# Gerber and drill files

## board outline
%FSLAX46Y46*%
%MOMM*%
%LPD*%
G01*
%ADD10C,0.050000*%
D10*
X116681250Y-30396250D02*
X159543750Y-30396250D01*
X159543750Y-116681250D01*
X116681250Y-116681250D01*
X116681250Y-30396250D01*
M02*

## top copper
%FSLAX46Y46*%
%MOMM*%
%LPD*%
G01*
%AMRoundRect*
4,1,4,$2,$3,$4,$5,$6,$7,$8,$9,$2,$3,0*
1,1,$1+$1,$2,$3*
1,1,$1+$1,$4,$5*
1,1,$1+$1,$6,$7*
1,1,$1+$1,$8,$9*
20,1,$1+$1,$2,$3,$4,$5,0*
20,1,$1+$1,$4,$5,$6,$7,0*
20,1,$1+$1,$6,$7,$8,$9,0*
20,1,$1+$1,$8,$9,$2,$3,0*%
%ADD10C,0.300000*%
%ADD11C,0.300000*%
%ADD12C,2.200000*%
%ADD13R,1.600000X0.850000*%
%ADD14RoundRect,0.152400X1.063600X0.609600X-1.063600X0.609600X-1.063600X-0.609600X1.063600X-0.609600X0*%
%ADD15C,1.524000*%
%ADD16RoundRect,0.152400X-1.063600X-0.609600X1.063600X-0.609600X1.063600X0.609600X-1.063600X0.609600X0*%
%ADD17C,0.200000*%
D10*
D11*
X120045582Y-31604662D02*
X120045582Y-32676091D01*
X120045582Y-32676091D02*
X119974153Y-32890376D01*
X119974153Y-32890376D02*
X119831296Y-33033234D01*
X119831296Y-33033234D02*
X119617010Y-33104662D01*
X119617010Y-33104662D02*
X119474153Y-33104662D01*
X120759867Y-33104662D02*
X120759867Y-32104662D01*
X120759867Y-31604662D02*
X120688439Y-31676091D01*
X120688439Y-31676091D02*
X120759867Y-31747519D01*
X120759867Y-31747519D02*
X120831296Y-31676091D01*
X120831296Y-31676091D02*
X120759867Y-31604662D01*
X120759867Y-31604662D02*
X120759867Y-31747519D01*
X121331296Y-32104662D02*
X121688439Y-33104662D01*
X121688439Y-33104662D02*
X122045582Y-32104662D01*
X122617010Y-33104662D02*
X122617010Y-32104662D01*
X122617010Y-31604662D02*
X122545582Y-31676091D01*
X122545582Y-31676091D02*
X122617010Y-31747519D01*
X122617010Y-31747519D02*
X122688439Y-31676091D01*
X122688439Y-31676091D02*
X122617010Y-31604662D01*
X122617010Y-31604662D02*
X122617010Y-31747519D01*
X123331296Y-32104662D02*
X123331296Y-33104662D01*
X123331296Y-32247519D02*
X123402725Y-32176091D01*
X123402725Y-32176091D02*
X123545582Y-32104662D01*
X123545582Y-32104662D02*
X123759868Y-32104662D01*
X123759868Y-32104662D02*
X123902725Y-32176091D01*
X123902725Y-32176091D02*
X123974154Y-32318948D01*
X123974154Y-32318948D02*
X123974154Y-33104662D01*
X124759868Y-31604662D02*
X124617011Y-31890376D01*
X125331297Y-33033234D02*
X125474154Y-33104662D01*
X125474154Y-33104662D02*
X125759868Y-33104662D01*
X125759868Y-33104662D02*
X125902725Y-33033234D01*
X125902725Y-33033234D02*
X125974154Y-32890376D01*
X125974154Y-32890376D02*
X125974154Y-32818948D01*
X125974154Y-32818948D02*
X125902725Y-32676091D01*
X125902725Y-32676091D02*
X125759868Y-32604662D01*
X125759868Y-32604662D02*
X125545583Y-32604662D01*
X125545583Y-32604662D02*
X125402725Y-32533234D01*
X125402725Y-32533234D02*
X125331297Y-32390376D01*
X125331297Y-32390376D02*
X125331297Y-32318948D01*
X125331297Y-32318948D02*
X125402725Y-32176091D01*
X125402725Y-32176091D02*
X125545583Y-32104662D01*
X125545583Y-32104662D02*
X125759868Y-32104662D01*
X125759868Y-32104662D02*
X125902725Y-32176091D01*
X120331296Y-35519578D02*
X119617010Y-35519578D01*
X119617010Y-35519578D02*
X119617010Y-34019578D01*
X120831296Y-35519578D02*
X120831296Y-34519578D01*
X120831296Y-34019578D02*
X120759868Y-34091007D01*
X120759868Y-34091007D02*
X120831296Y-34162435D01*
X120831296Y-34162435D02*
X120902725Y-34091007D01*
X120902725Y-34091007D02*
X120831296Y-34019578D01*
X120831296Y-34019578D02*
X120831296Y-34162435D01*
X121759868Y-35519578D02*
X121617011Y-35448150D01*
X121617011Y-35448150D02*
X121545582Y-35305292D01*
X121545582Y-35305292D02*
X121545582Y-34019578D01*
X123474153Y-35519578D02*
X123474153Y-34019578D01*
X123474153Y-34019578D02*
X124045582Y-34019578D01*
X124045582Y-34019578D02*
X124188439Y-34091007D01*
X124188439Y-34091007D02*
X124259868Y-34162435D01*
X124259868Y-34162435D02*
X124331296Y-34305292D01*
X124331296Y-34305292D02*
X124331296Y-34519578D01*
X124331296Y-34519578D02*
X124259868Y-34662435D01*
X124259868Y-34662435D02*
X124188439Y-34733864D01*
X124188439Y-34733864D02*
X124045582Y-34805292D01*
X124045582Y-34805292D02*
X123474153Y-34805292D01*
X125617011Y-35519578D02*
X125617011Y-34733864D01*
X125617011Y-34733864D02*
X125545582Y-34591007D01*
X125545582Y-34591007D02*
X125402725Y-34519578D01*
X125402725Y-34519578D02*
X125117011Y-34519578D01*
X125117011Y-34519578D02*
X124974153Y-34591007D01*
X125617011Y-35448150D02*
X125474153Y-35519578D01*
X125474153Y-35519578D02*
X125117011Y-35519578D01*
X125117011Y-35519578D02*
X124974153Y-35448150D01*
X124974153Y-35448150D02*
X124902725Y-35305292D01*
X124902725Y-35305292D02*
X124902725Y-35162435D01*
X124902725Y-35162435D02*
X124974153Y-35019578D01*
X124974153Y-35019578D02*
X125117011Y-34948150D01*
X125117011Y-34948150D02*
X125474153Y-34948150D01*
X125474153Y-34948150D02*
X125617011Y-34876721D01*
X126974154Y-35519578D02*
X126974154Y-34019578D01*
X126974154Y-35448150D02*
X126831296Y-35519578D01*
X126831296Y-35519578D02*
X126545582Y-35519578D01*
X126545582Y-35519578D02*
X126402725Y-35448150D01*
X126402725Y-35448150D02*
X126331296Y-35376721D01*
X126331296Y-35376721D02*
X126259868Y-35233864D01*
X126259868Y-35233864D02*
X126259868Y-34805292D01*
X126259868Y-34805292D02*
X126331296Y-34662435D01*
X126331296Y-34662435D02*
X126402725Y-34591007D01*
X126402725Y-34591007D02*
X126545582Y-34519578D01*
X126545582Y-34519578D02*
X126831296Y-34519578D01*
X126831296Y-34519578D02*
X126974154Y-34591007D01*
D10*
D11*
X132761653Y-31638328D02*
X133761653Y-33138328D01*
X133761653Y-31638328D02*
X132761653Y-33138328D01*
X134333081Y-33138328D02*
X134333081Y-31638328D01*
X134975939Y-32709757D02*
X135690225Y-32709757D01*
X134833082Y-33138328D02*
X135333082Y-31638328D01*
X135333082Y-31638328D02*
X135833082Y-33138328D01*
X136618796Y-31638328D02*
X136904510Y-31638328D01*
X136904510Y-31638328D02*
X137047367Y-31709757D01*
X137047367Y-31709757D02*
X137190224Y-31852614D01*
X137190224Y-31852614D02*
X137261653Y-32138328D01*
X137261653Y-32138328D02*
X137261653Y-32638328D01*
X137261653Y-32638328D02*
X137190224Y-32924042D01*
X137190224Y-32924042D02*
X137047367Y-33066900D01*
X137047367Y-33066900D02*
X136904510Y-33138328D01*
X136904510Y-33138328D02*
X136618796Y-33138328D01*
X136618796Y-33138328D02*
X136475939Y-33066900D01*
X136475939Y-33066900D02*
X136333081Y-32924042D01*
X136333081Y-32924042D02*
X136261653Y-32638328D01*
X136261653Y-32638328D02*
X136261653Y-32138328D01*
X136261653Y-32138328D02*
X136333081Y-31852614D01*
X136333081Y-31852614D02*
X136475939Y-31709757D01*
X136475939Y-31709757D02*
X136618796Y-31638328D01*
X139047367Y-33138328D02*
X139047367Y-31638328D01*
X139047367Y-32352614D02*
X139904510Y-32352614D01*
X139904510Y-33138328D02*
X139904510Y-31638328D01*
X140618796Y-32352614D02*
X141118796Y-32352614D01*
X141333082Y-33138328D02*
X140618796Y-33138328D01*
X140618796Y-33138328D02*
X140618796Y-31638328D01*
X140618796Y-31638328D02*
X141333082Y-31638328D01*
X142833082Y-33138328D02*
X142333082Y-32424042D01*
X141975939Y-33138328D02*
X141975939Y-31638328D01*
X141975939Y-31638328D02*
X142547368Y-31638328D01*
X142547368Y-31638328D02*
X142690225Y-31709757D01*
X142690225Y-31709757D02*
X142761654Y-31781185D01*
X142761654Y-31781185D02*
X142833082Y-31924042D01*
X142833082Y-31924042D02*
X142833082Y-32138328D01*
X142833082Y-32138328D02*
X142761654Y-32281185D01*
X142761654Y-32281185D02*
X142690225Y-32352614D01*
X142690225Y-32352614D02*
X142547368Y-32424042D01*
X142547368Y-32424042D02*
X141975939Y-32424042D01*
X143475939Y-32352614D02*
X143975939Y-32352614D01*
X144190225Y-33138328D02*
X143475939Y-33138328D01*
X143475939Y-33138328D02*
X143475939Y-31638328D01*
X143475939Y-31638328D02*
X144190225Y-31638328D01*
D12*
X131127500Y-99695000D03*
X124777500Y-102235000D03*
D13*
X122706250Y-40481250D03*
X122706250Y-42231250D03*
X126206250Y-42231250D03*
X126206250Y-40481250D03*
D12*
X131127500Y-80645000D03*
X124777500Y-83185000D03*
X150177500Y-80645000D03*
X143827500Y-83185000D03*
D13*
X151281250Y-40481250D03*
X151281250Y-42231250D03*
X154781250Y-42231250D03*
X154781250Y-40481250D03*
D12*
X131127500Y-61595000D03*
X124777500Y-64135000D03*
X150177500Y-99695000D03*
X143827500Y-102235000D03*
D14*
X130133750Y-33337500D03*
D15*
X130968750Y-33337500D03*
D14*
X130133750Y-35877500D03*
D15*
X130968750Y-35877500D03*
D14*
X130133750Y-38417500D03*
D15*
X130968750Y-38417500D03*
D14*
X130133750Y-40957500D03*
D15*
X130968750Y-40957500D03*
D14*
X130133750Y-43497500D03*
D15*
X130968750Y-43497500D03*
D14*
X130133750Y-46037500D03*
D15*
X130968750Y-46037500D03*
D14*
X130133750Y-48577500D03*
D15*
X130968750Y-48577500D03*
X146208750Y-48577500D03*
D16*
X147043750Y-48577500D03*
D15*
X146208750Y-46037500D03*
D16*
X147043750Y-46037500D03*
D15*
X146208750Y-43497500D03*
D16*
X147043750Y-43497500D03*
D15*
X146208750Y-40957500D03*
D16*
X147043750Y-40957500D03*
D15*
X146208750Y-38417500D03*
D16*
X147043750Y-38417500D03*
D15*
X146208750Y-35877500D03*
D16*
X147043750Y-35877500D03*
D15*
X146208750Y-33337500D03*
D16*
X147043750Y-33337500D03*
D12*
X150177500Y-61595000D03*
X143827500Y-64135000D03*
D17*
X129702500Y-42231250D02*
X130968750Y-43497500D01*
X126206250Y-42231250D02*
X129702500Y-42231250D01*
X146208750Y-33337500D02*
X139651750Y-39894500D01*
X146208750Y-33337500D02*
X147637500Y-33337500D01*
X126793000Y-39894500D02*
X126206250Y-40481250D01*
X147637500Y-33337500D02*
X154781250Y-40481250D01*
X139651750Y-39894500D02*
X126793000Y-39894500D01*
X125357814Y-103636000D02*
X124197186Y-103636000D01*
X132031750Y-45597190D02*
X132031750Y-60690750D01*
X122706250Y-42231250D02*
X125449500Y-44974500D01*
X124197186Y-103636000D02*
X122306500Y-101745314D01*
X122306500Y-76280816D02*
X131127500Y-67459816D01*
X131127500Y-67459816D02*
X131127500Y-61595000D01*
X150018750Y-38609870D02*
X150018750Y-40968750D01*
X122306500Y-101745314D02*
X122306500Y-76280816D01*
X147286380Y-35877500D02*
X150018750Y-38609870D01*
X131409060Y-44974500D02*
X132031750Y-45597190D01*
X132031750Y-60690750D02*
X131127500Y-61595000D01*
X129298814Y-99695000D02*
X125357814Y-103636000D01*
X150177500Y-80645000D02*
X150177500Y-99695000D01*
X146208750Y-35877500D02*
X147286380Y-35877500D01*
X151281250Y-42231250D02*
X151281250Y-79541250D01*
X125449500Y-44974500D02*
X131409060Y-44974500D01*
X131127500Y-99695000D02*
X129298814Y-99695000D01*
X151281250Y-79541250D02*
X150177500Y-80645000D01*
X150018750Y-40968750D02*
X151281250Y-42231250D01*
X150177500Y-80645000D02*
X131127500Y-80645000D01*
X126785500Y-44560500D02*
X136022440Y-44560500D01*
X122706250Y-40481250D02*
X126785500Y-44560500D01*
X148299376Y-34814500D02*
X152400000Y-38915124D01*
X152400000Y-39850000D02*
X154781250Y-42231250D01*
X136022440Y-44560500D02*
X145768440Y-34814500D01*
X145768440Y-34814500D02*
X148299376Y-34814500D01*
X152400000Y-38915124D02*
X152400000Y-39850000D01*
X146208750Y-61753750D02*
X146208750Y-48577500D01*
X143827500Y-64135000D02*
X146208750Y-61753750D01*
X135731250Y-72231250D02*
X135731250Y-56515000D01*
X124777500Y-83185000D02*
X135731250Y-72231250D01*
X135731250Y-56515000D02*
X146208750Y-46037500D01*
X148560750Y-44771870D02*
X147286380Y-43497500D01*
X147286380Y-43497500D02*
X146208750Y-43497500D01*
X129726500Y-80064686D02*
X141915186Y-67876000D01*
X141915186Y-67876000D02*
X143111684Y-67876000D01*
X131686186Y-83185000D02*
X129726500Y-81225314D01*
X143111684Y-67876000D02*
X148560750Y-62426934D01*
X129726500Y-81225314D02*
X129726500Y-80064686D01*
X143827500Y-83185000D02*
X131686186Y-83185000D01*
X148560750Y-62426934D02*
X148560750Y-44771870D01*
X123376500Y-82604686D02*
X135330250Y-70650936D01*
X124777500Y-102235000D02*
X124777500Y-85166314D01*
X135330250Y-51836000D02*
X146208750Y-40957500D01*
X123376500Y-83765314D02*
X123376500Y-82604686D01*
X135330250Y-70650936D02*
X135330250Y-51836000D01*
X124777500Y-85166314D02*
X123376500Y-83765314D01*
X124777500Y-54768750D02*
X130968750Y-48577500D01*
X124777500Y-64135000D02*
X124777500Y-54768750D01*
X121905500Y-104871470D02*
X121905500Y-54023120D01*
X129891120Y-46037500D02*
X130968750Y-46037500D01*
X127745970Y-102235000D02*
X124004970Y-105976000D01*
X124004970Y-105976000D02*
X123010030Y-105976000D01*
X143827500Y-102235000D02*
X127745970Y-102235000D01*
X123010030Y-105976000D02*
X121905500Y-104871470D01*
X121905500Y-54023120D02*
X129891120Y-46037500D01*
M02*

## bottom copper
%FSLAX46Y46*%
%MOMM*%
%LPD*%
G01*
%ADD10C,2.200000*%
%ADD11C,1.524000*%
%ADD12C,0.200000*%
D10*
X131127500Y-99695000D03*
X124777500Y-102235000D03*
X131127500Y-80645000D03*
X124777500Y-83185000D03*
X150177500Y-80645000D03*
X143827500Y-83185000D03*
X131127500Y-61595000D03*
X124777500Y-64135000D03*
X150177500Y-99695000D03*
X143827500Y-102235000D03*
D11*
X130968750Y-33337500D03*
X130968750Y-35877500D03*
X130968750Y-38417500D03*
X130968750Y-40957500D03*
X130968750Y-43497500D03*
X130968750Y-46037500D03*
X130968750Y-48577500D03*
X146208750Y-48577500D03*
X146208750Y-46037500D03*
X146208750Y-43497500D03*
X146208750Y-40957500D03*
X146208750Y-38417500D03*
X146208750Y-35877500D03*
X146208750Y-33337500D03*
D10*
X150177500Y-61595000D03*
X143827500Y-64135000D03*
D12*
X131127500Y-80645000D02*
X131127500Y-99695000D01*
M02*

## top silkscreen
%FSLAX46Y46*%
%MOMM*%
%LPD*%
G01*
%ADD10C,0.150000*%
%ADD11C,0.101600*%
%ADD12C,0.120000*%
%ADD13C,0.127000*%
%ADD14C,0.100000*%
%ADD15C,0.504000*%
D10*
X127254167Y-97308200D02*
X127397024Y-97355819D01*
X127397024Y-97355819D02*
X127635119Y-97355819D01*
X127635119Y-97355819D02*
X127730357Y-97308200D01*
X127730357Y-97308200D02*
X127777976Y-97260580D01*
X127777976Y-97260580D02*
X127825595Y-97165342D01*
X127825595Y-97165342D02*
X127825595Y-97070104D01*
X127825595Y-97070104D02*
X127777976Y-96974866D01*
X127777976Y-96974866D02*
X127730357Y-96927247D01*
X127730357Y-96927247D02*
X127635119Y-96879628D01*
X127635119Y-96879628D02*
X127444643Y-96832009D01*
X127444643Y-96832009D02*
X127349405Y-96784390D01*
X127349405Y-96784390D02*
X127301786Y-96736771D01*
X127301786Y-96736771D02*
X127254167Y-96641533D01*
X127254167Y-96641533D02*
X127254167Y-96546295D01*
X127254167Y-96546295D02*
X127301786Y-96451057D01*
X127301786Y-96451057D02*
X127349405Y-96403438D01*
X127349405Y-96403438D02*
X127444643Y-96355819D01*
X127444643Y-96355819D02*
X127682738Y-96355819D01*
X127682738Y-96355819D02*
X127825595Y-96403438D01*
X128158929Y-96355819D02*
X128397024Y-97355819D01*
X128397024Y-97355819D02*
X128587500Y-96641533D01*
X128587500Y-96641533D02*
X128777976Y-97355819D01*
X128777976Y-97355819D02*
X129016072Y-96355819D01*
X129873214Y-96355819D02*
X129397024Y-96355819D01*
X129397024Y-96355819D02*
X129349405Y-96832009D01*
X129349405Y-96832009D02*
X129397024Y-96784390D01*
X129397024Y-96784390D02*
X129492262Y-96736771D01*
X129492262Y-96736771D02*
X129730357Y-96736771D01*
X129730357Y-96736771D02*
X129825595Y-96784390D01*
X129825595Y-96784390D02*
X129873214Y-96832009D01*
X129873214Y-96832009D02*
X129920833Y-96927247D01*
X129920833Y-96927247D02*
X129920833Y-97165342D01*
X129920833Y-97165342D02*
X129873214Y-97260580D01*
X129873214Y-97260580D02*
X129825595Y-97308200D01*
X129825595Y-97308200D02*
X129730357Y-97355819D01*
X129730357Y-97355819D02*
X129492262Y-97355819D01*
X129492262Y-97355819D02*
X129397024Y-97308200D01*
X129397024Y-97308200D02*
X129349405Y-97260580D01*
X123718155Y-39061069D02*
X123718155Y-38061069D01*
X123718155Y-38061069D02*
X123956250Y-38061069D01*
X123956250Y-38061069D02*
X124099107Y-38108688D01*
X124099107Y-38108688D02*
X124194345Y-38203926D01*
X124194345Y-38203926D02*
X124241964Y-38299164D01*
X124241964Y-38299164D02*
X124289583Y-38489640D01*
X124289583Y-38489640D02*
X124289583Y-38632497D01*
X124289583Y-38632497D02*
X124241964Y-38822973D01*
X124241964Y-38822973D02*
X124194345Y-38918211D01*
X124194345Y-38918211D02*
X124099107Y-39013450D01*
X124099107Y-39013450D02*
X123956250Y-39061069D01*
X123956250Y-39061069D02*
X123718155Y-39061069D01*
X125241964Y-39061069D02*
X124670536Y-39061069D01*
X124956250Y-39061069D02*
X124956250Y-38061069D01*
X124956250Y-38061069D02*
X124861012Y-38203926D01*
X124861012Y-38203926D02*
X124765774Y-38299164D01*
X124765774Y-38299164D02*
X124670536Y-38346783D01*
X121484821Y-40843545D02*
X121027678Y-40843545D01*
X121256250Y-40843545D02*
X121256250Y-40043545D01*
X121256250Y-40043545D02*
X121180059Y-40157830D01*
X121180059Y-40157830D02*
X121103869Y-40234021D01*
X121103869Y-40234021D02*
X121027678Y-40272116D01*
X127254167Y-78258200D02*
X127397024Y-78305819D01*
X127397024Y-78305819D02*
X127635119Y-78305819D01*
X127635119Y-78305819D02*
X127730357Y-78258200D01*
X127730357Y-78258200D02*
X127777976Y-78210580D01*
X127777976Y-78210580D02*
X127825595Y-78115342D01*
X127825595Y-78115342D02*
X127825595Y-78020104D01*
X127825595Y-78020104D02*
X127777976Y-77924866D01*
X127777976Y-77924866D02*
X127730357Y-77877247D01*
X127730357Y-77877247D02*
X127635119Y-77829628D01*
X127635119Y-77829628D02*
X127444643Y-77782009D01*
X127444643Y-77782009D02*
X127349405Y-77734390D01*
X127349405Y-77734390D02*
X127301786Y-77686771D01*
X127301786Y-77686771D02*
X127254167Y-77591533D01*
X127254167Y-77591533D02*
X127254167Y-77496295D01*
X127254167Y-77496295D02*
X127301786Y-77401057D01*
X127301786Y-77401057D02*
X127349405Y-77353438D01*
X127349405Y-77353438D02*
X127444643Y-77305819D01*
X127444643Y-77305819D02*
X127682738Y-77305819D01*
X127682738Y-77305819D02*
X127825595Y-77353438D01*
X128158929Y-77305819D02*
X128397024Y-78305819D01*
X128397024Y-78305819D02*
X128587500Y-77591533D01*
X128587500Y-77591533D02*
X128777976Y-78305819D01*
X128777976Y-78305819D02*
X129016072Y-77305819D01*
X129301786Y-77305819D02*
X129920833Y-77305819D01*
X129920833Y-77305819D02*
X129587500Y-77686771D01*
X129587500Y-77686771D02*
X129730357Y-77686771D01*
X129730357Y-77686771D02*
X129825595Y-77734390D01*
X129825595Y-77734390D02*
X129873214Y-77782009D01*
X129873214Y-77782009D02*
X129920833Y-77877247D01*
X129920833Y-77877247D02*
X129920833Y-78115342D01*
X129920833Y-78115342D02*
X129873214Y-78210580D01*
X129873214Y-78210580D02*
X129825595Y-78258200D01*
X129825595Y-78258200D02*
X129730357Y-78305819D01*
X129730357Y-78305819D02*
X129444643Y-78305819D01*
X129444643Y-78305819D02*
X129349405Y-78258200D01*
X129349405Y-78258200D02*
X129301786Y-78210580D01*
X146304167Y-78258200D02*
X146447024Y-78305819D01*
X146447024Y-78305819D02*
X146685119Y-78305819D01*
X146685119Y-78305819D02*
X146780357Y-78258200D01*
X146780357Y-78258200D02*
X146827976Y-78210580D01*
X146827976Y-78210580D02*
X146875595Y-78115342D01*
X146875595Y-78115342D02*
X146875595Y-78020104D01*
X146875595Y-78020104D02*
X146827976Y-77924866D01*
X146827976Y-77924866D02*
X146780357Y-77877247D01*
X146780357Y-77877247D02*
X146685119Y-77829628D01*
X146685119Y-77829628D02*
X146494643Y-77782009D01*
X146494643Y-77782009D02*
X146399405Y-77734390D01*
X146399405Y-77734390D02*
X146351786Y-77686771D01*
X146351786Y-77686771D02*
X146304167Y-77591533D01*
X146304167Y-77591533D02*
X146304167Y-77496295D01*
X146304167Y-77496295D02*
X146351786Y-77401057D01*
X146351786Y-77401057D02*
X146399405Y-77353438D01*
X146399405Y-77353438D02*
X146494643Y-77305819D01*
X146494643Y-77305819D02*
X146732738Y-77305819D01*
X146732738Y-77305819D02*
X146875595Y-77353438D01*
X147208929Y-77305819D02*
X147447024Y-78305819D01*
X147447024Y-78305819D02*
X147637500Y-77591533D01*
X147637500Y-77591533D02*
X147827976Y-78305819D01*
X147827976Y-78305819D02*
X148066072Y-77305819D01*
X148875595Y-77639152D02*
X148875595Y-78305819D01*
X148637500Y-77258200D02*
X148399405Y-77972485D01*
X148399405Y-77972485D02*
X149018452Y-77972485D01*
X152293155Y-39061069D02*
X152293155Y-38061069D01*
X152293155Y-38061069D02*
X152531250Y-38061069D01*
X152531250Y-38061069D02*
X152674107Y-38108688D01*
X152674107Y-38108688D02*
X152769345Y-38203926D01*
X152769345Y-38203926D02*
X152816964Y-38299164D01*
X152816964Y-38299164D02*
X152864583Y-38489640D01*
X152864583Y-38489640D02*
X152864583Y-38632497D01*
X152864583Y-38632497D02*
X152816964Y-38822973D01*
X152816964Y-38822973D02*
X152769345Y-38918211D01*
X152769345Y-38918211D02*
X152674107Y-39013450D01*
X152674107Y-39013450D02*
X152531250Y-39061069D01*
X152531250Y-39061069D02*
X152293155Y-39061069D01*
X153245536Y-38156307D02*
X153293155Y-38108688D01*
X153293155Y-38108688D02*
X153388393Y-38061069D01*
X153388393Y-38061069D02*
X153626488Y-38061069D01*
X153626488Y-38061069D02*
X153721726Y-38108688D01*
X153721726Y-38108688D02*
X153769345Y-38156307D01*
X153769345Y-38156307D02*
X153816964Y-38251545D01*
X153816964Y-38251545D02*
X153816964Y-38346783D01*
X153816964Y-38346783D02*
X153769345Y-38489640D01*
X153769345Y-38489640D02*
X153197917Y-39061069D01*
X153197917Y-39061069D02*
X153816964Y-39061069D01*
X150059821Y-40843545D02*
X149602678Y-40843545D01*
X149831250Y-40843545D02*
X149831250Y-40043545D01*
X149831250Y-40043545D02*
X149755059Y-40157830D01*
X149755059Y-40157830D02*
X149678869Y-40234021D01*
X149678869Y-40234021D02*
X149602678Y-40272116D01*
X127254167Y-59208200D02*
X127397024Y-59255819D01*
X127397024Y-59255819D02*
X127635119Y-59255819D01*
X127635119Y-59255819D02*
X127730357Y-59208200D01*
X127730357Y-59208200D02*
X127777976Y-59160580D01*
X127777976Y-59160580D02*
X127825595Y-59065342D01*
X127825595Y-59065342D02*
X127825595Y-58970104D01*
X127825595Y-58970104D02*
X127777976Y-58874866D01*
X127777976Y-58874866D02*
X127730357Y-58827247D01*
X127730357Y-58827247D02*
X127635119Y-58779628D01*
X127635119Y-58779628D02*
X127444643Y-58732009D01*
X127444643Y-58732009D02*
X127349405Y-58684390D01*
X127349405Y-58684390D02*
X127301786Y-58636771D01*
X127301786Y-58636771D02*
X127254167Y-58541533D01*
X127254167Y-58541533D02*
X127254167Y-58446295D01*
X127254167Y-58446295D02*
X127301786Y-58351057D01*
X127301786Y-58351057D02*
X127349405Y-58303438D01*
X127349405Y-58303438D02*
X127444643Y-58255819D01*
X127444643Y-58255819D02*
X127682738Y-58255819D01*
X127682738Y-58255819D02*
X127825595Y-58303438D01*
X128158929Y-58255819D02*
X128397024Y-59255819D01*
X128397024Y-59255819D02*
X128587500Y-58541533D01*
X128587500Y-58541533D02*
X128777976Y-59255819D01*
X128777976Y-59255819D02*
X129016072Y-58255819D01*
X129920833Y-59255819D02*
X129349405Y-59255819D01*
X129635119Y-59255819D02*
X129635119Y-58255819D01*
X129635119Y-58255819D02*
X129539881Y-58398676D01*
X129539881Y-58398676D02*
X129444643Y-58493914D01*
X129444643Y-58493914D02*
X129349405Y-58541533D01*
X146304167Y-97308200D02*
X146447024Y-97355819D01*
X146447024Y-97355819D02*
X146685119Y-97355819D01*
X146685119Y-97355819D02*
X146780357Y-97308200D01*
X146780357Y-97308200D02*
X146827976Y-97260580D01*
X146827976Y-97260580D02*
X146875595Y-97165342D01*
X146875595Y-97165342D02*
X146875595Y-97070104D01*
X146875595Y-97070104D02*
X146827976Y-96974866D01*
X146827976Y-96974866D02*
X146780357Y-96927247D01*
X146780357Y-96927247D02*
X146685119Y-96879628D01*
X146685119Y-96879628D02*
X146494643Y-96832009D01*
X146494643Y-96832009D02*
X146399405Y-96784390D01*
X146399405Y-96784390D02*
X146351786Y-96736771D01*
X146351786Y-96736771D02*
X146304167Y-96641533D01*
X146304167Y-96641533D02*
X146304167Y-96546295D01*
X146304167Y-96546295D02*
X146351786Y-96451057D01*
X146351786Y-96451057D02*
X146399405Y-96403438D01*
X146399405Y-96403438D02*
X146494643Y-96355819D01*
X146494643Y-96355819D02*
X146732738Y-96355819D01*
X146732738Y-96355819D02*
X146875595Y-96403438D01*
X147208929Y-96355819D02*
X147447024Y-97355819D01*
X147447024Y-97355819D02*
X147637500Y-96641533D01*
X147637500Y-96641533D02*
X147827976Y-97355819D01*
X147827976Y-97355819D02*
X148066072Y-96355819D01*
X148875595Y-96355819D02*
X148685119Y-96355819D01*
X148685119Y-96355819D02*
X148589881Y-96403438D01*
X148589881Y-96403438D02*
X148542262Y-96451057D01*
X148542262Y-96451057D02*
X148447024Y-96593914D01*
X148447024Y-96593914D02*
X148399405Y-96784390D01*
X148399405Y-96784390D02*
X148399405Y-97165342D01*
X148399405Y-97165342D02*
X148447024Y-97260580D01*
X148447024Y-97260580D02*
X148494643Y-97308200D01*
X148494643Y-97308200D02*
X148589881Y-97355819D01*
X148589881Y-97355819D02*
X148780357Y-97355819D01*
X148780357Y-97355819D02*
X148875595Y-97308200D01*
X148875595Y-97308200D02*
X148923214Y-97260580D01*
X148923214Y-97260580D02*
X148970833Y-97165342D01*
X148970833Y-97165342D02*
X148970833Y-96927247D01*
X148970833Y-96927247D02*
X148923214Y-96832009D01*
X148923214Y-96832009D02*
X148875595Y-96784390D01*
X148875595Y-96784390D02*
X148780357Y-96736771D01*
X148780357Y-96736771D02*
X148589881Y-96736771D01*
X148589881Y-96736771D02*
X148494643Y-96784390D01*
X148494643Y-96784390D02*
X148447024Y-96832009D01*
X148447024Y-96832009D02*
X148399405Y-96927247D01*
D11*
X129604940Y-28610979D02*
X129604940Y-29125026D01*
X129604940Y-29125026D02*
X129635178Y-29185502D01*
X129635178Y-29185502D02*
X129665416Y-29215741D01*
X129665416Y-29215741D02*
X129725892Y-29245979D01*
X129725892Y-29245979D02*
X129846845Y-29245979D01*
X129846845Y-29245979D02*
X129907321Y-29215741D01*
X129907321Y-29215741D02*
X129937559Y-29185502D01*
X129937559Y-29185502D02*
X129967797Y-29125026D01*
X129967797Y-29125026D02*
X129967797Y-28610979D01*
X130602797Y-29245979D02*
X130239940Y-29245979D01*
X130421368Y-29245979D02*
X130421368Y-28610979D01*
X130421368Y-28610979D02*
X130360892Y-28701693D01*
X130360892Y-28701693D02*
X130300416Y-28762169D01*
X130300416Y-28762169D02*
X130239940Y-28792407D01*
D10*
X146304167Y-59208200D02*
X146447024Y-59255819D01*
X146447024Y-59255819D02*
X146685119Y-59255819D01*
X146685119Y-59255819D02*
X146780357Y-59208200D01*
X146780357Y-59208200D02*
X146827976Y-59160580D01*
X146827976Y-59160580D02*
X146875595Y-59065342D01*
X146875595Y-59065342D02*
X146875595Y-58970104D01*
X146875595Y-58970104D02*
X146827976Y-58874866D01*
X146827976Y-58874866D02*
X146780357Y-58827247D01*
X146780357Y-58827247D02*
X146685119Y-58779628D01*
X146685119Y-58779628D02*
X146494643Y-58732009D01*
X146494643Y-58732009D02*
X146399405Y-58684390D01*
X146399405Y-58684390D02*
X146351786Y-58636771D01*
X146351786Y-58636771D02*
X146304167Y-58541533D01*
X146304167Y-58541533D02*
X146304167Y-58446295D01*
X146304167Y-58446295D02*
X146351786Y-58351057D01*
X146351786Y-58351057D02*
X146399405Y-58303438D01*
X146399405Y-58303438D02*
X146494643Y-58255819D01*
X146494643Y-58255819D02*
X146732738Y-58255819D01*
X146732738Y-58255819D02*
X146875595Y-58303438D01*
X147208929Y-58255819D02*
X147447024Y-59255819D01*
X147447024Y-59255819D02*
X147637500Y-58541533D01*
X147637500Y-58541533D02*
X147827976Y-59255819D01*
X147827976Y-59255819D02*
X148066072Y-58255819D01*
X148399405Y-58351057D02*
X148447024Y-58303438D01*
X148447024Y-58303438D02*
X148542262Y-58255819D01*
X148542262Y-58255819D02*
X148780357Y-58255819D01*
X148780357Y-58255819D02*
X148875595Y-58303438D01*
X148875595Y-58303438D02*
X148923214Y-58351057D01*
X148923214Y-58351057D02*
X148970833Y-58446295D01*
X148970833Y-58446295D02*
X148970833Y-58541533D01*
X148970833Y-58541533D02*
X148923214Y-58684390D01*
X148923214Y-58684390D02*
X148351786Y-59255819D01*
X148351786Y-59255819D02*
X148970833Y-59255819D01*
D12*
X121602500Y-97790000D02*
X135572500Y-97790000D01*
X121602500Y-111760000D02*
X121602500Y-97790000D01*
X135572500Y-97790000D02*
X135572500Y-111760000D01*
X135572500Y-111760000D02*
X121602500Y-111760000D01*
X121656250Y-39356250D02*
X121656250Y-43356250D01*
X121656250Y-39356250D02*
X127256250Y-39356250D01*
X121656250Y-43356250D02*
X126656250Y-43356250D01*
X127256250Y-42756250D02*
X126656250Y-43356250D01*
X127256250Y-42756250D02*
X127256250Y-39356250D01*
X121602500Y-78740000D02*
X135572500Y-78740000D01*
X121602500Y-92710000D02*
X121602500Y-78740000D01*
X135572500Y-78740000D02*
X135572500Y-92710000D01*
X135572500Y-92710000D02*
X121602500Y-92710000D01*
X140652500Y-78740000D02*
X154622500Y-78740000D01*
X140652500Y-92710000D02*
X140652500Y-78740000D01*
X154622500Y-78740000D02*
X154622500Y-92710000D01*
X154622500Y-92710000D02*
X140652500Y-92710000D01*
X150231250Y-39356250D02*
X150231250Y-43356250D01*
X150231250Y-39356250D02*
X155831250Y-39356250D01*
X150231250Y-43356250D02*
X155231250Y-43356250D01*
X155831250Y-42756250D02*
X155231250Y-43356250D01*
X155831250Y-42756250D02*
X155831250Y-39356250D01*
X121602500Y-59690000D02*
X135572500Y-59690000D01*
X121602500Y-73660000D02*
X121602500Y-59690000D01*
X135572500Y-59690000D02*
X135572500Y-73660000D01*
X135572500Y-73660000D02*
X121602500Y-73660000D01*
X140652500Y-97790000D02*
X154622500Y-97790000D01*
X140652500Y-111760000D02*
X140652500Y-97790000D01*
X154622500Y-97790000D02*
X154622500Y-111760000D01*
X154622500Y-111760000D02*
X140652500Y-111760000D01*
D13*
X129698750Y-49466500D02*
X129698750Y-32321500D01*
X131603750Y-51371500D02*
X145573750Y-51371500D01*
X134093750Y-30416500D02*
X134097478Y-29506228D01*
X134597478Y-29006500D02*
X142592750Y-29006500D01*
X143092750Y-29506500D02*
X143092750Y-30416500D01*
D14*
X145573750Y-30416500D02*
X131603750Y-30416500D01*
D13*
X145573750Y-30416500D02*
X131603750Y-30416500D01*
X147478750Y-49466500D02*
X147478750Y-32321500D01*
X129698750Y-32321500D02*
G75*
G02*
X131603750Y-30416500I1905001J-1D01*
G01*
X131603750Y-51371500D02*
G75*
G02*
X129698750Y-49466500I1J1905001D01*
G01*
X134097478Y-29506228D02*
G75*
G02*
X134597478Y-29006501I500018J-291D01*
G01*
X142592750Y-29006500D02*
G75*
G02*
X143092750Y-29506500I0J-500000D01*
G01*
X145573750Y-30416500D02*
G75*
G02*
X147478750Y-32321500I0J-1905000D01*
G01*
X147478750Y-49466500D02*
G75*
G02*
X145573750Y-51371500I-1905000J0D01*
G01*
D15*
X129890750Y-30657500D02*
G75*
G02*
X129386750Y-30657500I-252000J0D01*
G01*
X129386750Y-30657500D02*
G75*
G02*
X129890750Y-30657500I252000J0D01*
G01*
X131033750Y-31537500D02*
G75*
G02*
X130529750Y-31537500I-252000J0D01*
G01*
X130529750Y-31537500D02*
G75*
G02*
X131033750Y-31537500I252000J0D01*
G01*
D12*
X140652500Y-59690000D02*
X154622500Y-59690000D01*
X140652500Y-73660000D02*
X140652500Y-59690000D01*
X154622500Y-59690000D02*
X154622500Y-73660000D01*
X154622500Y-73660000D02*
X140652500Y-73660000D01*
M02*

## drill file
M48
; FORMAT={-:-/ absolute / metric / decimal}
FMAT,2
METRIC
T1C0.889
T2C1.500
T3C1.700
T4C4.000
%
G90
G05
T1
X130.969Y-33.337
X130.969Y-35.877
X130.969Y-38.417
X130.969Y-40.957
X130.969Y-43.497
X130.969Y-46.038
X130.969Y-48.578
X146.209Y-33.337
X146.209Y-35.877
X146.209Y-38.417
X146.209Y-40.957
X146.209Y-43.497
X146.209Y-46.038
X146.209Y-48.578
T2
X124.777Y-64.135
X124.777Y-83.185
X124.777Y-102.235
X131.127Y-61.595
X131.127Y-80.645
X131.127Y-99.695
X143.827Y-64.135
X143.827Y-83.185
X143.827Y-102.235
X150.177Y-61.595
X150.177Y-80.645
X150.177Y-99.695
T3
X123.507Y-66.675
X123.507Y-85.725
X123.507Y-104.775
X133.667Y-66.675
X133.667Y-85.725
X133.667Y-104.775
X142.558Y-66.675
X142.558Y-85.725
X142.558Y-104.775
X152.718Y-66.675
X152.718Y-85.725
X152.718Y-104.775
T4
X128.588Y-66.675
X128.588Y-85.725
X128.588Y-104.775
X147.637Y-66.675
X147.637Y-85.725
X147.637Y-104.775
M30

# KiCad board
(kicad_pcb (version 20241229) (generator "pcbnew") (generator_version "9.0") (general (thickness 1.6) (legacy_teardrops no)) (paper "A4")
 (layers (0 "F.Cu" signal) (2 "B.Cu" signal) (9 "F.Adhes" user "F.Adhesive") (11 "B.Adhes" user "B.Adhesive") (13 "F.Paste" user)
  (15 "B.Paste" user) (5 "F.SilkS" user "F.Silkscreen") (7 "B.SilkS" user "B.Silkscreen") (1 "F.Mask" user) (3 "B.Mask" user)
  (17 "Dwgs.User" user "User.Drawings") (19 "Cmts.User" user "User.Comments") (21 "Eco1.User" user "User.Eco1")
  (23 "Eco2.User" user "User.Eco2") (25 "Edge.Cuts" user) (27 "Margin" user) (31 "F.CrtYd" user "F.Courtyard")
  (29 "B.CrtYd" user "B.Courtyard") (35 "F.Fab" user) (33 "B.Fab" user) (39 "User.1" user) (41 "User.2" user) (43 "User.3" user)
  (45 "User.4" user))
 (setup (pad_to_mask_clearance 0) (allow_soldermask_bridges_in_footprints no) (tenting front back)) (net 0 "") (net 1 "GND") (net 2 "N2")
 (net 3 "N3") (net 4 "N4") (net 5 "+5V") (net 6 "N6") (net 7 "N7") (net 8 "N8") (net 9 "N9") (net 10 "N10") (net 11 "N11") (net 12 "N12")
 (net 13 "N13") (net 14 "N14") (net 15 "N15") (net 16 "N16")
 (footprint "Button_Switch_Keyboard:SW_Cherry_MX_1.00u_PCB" (layer "F.Cu") (at 131.1275 99.695)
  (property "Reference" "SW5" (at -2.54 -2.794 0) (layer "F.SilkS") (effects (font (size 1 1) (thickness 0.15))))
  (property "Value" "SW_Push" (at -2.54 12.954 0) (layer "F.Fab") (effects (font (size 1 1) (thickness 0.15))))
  (fp_line (start -9.525 -1.905) (end 4.445 -1.905) (stroke (width 0.12) (type solid)) (layer "F.SilkS"))
  (fp_line (start -9.525 12.065) (end -9.525 -1.905) (stroke (width 0.12) (type solid)) (layer "F.SilkS"))
  (fp_line (start 4.445 -1.905) (end 4.445 12.065) (stroke (width 0.12) (type solid)) (layer "F.SilkS"))
  (fp_line (start 4.445 12.065) (end -9.525 12.065) (stroke (width 0.12) (type solid)) (layer "F.SilkS"))
  (pad "" np_thru_hole circle (at -7.62 5.08) (size 1.7 1.7) (drill 1.7) (layers "*.Cu" "*.Mask"))
  (pad "" np_thru_hole circle (at -2.54 5.08) (size 4 4) (drill 4) (layers "*.Cu" "*.Mask"))
  (pad "" np_thru_hole circle (at 2.54 5.08) (size 1.7 1.7) (drill 1.7) (layers "*.Cu" "*.Mask"))
  (pad "1" thru_hole circle (at 0 0) (size 2.2 2.2) (drill 1.5) (layers "*.Cu" "*.Mask") (remove_unused_layers no) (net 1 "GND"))
  (pad "2" thru_hole circle (at -6.35 2.54) (size 2.2 2.2) (drill 1.5) (layers "*.Cu" "*.Mask") (remove_unused_layers no) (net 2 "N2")))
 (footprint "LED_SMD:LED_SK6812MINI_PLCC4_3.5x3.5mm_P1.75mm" (layer "F.Cu") (at 124.45625 41.35625)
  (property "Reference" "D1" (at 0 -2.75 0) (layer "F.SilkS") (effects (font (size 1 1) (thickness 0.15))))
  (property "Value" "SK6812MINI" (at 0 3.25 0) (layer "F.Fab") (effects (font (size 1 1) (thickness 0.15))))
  (fp_line (start -2.8 -2) (end -2.8 2) (stroke (width 0.12) (type default)) (layer "F.SilkS"))
  (fp_line (start -2.8 -2) (end 2.8 -2) (stroke (width 0.12) (type solid)) (layer "F.SilkS"))
  (fp_line (start -2.8 2) (end 2.2 2) (stroke (width 0.12) (type solid)) (layer "F.SilkS"))
  (fp_line (start 2.8 1.4) (end 2.2 2) (stroke (width 0.12) (type default)) (layer "F.SilkS"))
  (fp_line (start 2.8 1.4) (end 2.8 -2) (stroke (width 0.12) (type solid)) (layer "F.SilkS"))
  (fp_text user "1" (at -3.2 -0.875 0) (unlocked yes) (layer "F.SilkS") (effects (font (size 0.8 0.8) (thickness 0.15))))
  (pad "1" smd rect (at -1.75 -0.875) (size 1.6 0.85) (layers "F.Cu" "F.Mask" "F.Paste") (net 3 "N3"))
  (pad "2" smd rect (at -1.75 0.875) (size 1.6 0.85) (layers "F.Cu" "F.Mask" "F.Paste") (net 1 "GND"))
  (pad "3" smd rect (at 1.75 0.875) (size 1.6 0.85) (layers "F.Cu" "F.Mask" "F.Paste") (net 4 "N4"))
  (pad "4" smd rect (at 1.75 -0.875) (size 1.6 0.85) (layers "F.Cu" "F.Mask" "F.Paste") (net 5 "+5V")))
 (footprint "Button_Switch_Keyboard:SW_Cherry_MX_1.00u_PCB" (layer "F.Cu") (at 131.1275 80.645)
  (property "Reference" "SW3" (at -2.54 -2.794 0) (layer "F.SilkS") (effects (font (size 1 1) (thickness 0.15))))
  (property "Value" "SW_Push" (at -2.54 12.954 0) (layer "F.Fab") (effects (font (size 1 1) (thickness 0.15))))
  (fp_line (start -9.525 -1.905) (end 4.445 -1.905) (stroke (width 0.12) (type solid)) (layer "F.SilkS"))
  (fp_line (start -9.525 12.065) (end -9.525 -1.905) (stroke (width 0.12) (type solid)) (layer "F.SilkS"))
  (fp_line (start 4.445 -1.905) (end 4.445 12.065) (stroke (width 0.12) (type solid)) (layer "F.SilkS"))
  (fp_line (start 4.445 12.065) (end -9.525 12.065) (stroke (width 0.12) (type solid)) (layer "F.SilkS"))
  (pad "" np_thru_hole circle (at -7.62 5.08) (size 1.7 1.7) (drill 1.7) (layers "*.Cu" "*.Mask"))
  (pad "" np_thru_hole circle (at -2.54 5.08) (size 4 4) (drill 4) (layers "*.Cu" "*.Mask"))
  (pad "" np_thru_hole circle (at 2.54 5.08) (size 1.7 1.7) (drill 1.7) (layers "*.Cu" "*.Mask"))
  (pad "1" thru_hole circle (at 0 0) (size 2.2 2.2) (drill 1.5) (layers "*.Cu" "*.Mask") (remove_unused_layers no) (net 1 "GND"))
  (pad "2" thru_hole circle (at -6.35 2.54) (size 2.2 2.2) (drill 1.5) (layers "*.Cu" "*.Mask") (remove_unused_layers no) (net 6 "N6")))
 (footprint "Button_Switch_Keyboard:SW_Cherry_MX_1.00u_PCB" (layer "F.Cu") (at 150.1775 80.645)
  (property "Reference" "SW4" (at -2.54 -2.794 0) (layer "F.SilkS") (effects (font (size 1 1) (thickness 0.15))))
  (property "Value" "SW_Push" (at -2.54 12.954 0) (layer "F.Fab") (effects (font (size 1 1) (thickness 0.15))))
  (fp_line (start -9.525 -1.905) (end 4.445 -1.905) (stroke (width 0.12) (type solid)) (layer "F.SilkS"))
  (fp_line (start -9.525 12.065) (end -9.525 -1.905) (stroke (width 0.12) (type solid)) (layer "F.SilkS"))
  (fp_line (start 4.445 -1.905) (end 4.445 12.065) (stroke (width 0.12) (type solid)) (layer "F.SilkS"))
  (fp_line (start 4.445 12.065) (end -9.525 12.065) (stroke (width 0.12) (type solid)) (layer "F.SilkS"))
  (pad "" np_thru_hole circle (at -7.62 5.08) (size 1.7 1.7) (drill 1.7) (layers "*.Cu" "*.Mask"))
  (pad "" np_thru_hole circle (at -2.54 5.08) (size 4 4) (drill 4) (layers "*.Cu" "*.Mask"))
  (pad "" np_thru_hole circle (at 2.54 5.08) (size 1.7 1.7) (drill 1.7) (layers "*.Cu" "*.Mask"))
  (pad "1" thru_hole circle (at 0 0) (size 2.2 2.2) (drill 1.5) (layers "*.Cu" "*.Mask") (remove_unused_layers no) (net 1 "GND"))
  (pad "2" thru_hole circle (at -6.35 2.54) (size 2.2 2.2) (drill 1.5) (layers "*.Cu" "*.Mask") (remove_unused_layers no) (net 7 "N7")))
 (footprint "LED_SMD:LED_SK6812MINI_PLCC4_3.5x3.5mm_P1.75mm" (layer "F.Cu") (at 153.03125 41.35625)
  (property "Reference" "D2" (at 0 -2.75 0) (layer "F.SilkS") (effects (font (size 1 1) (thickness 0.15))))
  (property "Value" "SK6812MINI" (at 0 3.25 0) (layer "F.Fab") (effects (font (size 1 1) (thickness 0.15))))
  (fp_line (start -2.8 -2) (end -2.8 2) (stroke (width 0.12) (type default)) (layer "F.SilkS"))
  (fp_line (start -2.8 -2) (end 2.8 -2) (stroke (width 0.12) (type solid)) (layer "F.SilkS"))
  (fp_line (start -2.8 2) (end 2.2 2) (stroke (width 0.12) (type solid)) (layer "F.SilkS"))
  (fp_line (start 2.8 1.4) (end 2.2 2) (stroke (width 0.12) (type default)) (layer "F.SilkS"))
  (fp_line (start 2.8 1.4) (end 2.8 -2) (stroke (width 0.12) (type solid)) (layer "F.SilkS"))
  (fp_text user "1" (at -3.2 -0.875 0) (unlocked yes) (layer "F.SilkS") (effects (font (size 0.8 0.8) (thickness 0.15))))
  (pad "1" smd rect (at -1.75 -0.875) (size 1.6 0.85) (layers "F.Cu" "F.Mask" "F.Paste") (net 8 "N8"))
  (pad "2" smd rect (at -1.75 0.875) (size 1.6 0.85) (layers "F.Cu" "F.Mask" "F.Paste") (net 1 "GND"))
  (pad "3" smd rect (at 1.75 0.875) (size 1.6 0.85) (layers "F.Cu" "F.Mask" "F.Paste") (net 3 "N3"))
  (pad "4" smd rect (at 1.75 -0.875) (size 1.6 0.85) (layers "F.Cu" "F.Mask" "F.Paste") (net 5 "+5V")))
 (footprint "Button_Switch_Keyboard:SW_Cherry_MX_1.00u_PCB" (layer "F.Cu") (at 131.1275 61.595)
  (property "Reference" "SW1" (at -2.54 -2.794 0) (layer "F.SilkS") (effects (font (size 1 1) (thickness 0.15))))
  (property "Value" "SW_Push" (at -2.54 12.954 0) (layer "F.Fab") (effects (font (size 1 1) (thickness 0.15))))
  (fp_line (start -9.525 -1.905) (end 4.445 -1.905) (stroke (width 0.12) (type solid)) (layer "F.SilkS"))
  (fp_line (start -9.525 12.065) (end -9.525 -1.905) (stroke (width 0.12) (type solid)) (layer "F.SilkS"))
  (fp_line (start 4.445 -1.905) (end 4.445 12.065) (stroke (width 0.12) (type solid)) (layer "F.SilkS"))
  (fp_line (start 4.445 12.065) (end -9.525 12.065) (stroke (width 0.12) (type solid)) (layer "F.SilkS"))
  (pad "" np_thru_hole circle (at -7.62 5.08) (size 1.7 1.7) (drill 1.7) (layers "*.Cu" "*.Mask"))
  (pad "" np_thru_hole circle (at -2.54 5.08) (size 4 4) (drill 4) (layers "*.Cu" "*.Mask"))
  (pad "" np_thru_hole circle (at 2.54 5.08) (size 1.7 1.7) (drill 1.7) (layers "*.Cu" "*.Mask"))
  (pad "1" thru_hole circle (at 0 0) (size 2.2 2.2) (drill 1.5) (layers "*.Cu" "*.Mask") (remove_unused_layers no) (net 1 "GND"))
  (pad "2" thru_hole circle (at -6.35 2.54) (size 2.2 2.2) (drill 1.5) (layers "*.Cu" "*.Mask") (remove_unused_layers no) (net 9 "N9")))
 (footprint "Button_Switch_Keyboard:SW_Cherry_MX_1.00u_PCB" (layer "F.Cu") (at 150.1775 99.695)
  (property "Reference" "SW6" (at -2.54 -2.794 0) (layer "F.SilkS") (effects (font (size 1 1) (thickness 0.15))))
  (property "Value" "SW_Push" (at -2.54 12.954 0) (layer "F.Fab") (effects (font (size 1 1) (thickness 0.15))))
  (fp_line (start -9.525 -1.905) (end 4.445 -1.905) (stroke (width 0.12) (type solid)) (layer "F.SilkS"))
  (fp_line (start -9.525 12.065) (end -9.525 -1.905) (stroke (width 0.12) (type solid)) (layer "F.SilkS"))
  (fp_line (start 4.445 -1.905) (end 4.445 12.065) (stroke (width 0.12) (type solid)) (layer "F.SilkS"))
  (fp_line (start 4.445 12.065) (end -9.525 12.065) (stroke (width 0.12) (type solid)) (layer "F.SilkS"))
  (pad "" np_thru_hole circle (at -7.62 5.08) (size 1.7 1.7) (drill 1.7) (layers "*.Cu" "*.Mask"))
  (pad "" np_thru_hole circle (at -2.54 5.08) (size 4 4) (drill 4) (layers "*.Cu" "*.Mask"))
  (pad "" np_thru_hole circle (at 2.54 5.08) (size 1.7 1.7) (drill 1.7) (layers "*.Cu" "*.Mask"))
  (pad "1" thru_hole circle (at 0 0) (size 2.2 2.2) (drill 1.5) (layers "*.Cu" "*.Mask") (remove_unused_layers no) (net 1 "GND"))
  (pad "2" thru_hole circle (at -6.35 2.54) (size 2.2 2.2) (drill 1.5) (layers "*.Cu" "*.Mask") (remove_unused_layers no) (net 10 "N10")))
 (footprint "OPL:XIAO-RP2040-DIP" (layer "F.Cu") (at 138.58875 40.9575)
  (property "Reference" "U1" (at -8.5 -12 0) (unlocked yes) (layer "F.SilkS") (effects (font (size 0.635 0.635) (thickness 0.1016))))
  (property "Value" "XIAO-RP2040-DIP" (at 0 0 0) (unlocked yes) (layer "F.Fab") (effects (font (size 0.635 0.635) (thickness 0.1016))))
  (fp_line (start -8.89 8.509) (end -8.89 -8.636) (stroke (width 0.127) (type solid)) (layer "F.SilkS"))
  (fp_line (start -6.985 10.414) (end 6.985 10.414) (stroke (width 0.127) (type solid)) (layer "F.SilkS"))
  (fp_line (start -4.495 -10.541) (end -4.491272 -11.451272) (stroke (width 0.127) (type solid)) (layer "F.SilkS"))
  (fp_line (start -3.991272 -11.951) (end 4.004 -11.951) (stroke (width 0.127) (type solid)) (layer "F.SilkS"))
  (fp_line (start 4.504 -11.451) (end 4.504 -10.541) (stroke (width 0.127) (type solid)) (layer "F.SilkS"))
  (fp_line (start 6.985 -10.541) (end -6.985 -10.541) (stroke (width 0.1) (type solid)) (layer "F.SilkS"))
  (fp_line (start 6.985 -10.541) (end -6.985 -10.541) (stroke (width 0.127) (type solid)) (layer "F.SilkS"))
  (fp_line (start 8.89 8.509) (end 8.89 -8.636) (stroke (width 0.127) (type solid)) (layer "F.SilkS"))
  (fp_arc (start -8.89 -8.636) (mid -8.332038 -9.983038) (end -6.985 -10.541) (stroke (width 0.127) (type solid)) (layer "F.SilkS"))
  (fp_arc (start -6.985 10.414) (mid -8.332038 9.856038) (end -8.89 8.509) (stroke (width 0.127) (type solid)) (layer "F.SilkS"))
  (fp_arc (start -4.491272 -11.451272) (mid -4.344728 -11.80464) (end -3.991272 -11.951) (stroke (width 0.127) (type default))
   (layer "F.SilkS"))
  (fp_arc (start 4.004 -11.951) (mid 4.357553 -11.804553) (end 4.504 -11.451) (stroke (width 0.127) (type default)) (layer "F.SilkS"))
  (fp_arc (start 6.985 -10.541) (mid 8.332038 -9.983038) (end 8.89 -8.636) (stroke (width 0.127) (type solid)) (layer "F.SilkS"))
  (fp_arc (start 8.89 8.509) (mid 8.332038 9.856038) (end 6.985 10.414) (stroke (width 0.127) (type solid)) (layer "F.SilkS"))
  (fp_circle (center -8.95 -10.3) (end -8.95 -10.554) (stroke (width 0.5) (type solid)) (fill yes) (layer "F.SilkS"))
  (fp_circle (center -7.807 -9.42) (end -7.807 -9.674) (stroke (width 0.5) (type solid)) (fill yes) (layer "F.SilkS"))
  (pad "1" smd roundrect (at -8.455 -7.62 180) (size 2.432 1.524) (layers "F.Cu" "F.Mask") (roundrect_rratio 0.1) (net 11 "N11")
   (thermal_bridge_angle 45))
  (pad "1" thru_hole circle (at -7.62 -7.62 180) (size 1.524 1.524) (drill 0.889) (layers "*.Cu" "*.Mask") (remove_unused_layers no)
   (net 11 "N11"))
  (pad "2" smd roundrect (at -8.455 -5.08 180) (size 2.432 1.524) (layers "F.Cu" "F.Mask") (roundrect_rratio 0.1) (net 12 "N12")
   (thermal_bridge_angle 45))
  (pad "2" thru_hole circle (at -7.62 -5.08 180) (size 1.524 1.524) (drill 0.889) (layers "*.Cu" "*.Mask") (remove_unused_layers no)
   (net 12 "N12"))
  (pad "3" smd roundrect (at -8.455 -2.54 180) (size 2.432 1.524) (layers "F.Cu" "F.Mask") (roundrect_rratio 0.1) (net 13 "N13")
   (thermal_bridge_angle 45))
  (pad "3" thru_hole circle (at -7.62 -2.54 180) (size 1.524 1.524) (drill 0.889) (layers "*.Cu" "*.Mask") (remove_unused_layers no)
   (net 13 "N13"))
  (pad "4" smd roundrect (at -8.455 0 180) (size 2.432 1.524) (layers "F.Cu" "F.Mask") (roundrect_rratio 0.1) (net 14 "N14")
   (thermal_bridge_angle 45))
  (pad "4" thru_hole circle (at -7.62 0 180) (size 1.524 1.524) (drill 0.889) (layers "*.Cu" "*.Mask") (remove_unused_layers no)
   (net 14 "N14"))
  (pad "5" smd roundrect (at -8.455 2.54 180) (size 2.432 1.524) (layers "F.Cu" "F.Mask") (roundrect_rratio 0.1) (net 4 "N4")
   (thermal_bridge_angle 45))
  (pad "5" thru_hole circle (at -7.62 2.54 180) (size 1.524 1.524) (drill 0.889) (layers "*.Cu" "*.Mask") (remove_unused_layers no)
   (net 4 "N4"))
  (pad "6" smd roundrect (at -8.455 5.08 180) (size 2.432 1.524) (layers "F.Cu" "F.Mask") (roundrect_rratio 0.1) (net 10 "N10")
   (thermal_bridge_angle 45))
  (pad "6" thru_hole circle (at -7.62 5.08 180) (size 1.524 1.524) (drill 0.889) (layers "*.Cu" "*.Mask") (remove_unused_layers no)
   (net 10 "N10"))
  (pad "7" smd roundrect (at -8.455 7.62 180) (size 2.432 1.524) (layers "F.Cu" "F.Mask") (roundrect_rratio 0.1) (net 9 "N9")
   (thermal_bridge_angle 45))
  (pad "7" thru_hole circle (at -7.62 7.62 180) (size 1.524 1.524) (drill 0.889) (layers "*.Cu" "*.Mask") (remove_unused_layers no)
   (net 9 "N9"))
  (pad "8" thru_hole circle (at 7.62 7.62) (size 1.524 1.524) (drill 0.889) (layers "*.Cu" "*.Mask") (remove_unused_layers no)
   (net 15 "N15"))
  (pad "8" smd roundrect (at 8.455 7.62) (size 2.432 1.524) (layers "F.Cu" "F.Mask") (roundrect_rratio 0.1) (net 15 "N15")
   (thermal_bridge_angle 45))
  (pad "9" thru_hole circle (at 7.62 5.08) (size 1.524 1.524) (drill 0.889) (layers "*.Cu" "*.Mask") (remove_unused_layers no) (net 6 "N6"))
  (pad "9" smd roundrect (at 8.455 5.08) (size 2.432 1.524) (layers "F.Cu" "F.Mask") (roundrect_rratio 0.1) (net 6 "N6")
   (thermal_bridge_angle 45))
  (pad "10" thru_hole circle (at 7.62 2.54) (size 1.524 1.524) (drill 0.889) (layers "*.Cu" "*.Mask") (remove_unused_layers no) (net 7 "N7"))
  (pad "10" smd roundrect (at 8.455 2.54) (size 2.432 1.524) (layers "F.Cu" "F.Mask") (roundrect_rratio 0.1) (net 7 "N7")
   (thermal_bridge_angle 45))
  (pad "11" thru_hole circle (at 7.62 0) (size 1.524 1.524) (drill 0.889) (layers "*.Cu" "*.Mask") (remove_unused_layers no) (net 2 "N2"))
  (pad "11" smd roundrect (at 8.455 0) (size 2.432 1.524) (layers "F.Cu" "F.Mask") (roundrect_rratio 0.1) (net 2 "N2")
   (thermal_bridge_angle 45))
  (pad "12" thru_hole circle (at 7.62 -2.54) (size 1.524 1.524) (drill 0.889) (layers "*.Cu" "*.Mask") (remove_unused_layers no)
   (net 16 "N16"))
  (pad "12" smd roundrect (at 8.455 -2.54) (size 2.432 1.524) (layers "F.Cu" "F.Mask") (roundrect_rratio 0.1) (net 16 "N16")
   (thermal_bridge_angle 45))
  (pad "13" thru_hole circle (at 7.62 -5.08) (size 1.524 1.524) (drill 0.889) (layers "*.Cu" "*.Mask") (remove_unused_layers no)
   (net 1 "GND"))
  (pad "13" smd roundrect (at 8.455 -5.08) (size 2.432 1.524) (layers "F.Cu" "F.Mask") (roundrect_rratio 0.1) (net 1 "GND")
   (thermal_bridge_angle 45))
  (pad "14" thru_hole circle (at 7.62 -7.62) (size 1.524 1.524) (drill 0.889) (layers "*.Cu" "*.Mask") (remove_unused_layers no)
   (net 5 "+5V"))
  (pad "14" smd roundrect (at 8.455 -7.62) (size 2.432 1.524) (layers "F.Cu" "F.Mask") (roundrect_rratio 0.1) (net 5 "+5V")
   (thermal_bridge_angle 45)))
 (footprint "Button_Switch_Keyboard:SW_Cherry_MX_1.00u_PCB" (layer "F.Cu") (at 150.1775 61.595)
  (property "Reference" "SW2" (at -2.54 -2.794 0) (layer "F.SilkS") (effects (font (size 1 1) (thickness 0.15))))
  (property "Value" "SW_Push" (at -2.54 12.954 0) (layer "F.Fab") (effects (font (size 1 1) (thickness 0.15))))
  (fp_line (start -9.525 -1.905) (end 4.445 -1.905) (stroke (width 0.12) (type solid)) (layer "F.SilkS"))
  (fp_line (start -9.525 12.065) (end -9.525 -1.905) (stroke (width 0.12) (type solid)) (layer "F.SilkS"))
  (fp_line (start 4.445 -1.905) (end 4.445 12.065) (stroke (width 0.12) (type solid)) (layer "F.SilkS"))
  (fp_line (start 4.445 12.065) (end -9.525 12.065) (stroke (width 0.12) (type solid)) (layer "F.SilkS"))
  (pad "" np_thru_hole circle (at -7.62 5.08) (size 1.7 1.7) (drill 1.7) (layers "*.Cu" "*.Mask"))
  (pad "" np_thru_hole circle (at -2.54 5.08) (size 4 4) (drill 4) (layers "*.Cu" "*.Mask"))
  (pad "" np_thru_hole circle (at 2.54 5.08) (size 1.7 1.7) (drill 1.7) (layers "*.Cu" "*.Mask"))
  (pad "1" thru_hole circle (at 0 0) (size 2.2 2.2) (drill 1.5) (layers "*.Cu" "*.Mask") (remove_unused_layers no) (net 1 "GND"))
  (pad "2" thru_hole circle (at -6.35 2.54) (size 2.2 2.2) (drill 1.5) (layers "*.Cu" "*.Mask") (remove_unused_layers no) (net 15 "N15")))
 (gr_rect (start 116.68125 30.39625) (end 159.54375 116.68125) (stroke (width 0.05) (type default)) (fill no) (layer "Edge.Cuts"))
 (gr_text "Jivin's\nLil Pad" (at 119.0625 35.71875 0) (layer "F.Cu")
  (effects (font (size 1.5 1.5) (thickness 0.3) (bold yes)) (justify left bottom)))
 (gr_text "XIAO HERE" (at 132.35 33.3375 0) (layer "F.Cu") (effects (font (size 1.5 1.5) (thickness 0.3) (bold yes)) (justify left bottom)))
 (segment (start 129.7025 42.23125) (end 130.96875 43.4975) (width 0.2) (layer "F.Cu") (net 4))
 (segment (start 126.20625 42.23125) (end 129.7025 42.23125) (width 0.2) (layer "F.Cu") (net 4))
 (segment (start 146.20875 33.3375) (end 139.65175 39.8945) (width 0.2) (layer "F.Cu") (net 5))
 (segment (start 146.20875 33.3375) (end 147.6375 33.3375) (width 0.2) (layer "F.Cu") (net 5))
 (segment (start 126.793 39.8945) (end 126.20625 40.48125) (width 0.2) (layer "F.Cu") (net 5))
 (segment (start 147.6375 33.3375) (end 154.78125 40.48125) (width 0.2) (layer "F.Cu") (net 5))
 (segment (start 139.65175 39.8945) (end 126.793 39.8945) (width 0.2) (layer "F.Cu") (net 5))
 (segment (start 125.357814 103.636) (end 124.197186 103.636) (width 0.2) (layer "F.Cu") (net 1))
 (segment (start 132.03175 45.59719) (end 132.03175 60.69075) (width 0.2) (layer "F.Cu") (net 1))
 (segment (start 122.70625 42.23125) (end 125.4495 44.9745) (width 0.2) (layer "F.Cu") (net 1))
 (segment (start 124.197186 103.636) (end 122.3065 101.745314) (width 0.2) (layer "F.Cu") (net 1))
 (segment (start 122.3065 76.280816) (end 131.1275 67.459816) (width 0.2) (layer "F.Cu") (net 1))
 (segment (start 131.1275 67.459816) (end 131.1275 61.595) (width 0.2) (layer "F.Cu") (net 1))
 (segment (start 150.01875 38.60987) (end 150.01875 40.96875) (width 0.2) (layer "F.Cu") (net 1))
 (segment (start 122.3065 101.745314) (end 122.3065 76.280816) (width 0.2) (layer "F.Cu") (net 1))
 (segment (start 147.28638 35.8775) (end 150.01875 38.60987) (width 0.2) (layer "F.Cu") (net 1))
 (segment (start 131.40906 44.9745) (end 132.03175 45.59719) (width 0.2) (layer "F.Cu") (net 1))
 (segment (start 132.03175 60.69075) (end 131.1275 61.595) (width 0.2) (layer "F.Cu") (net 1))
 (segment (start 129.298814 99.695) (end 125.357814 103.636) (width 0.2) (layer "F.Cu") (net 1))
 (segment (start 150.1775 80.645) (end 150.1775 99.695) (width 0.2) (layer "F.Cu") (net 1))
 (segment (start 146.20875 35.8775) (end 147.28638 35.8775) (width 0.2) (layer "F.Cu") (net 1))
 (segment (start 151.28125 42.23125) (end 151.28125 79.54125) (width 0.2) (layer "F.Cu") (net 1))
 (segment (start 125.4495 44.9745) (end 131.40906 44.9745) (width 0.2) (layer "F.Cu") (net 1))
 (segment (start 131.1275 99.695) (end 129.298814 99.695) (width 0.2) (layer "F.Cu") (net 1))
 (segment (start 151.28125 79.54125) (end 150.1775 80.645) (width 0.2) (layer "F.Cu") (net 1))
 (segment (start 150.01875 40.96875) (end 151.28125 42.23125) (width 0.2) (layer "F.Cu") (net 1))
 (segment (start 150.1775 80.645) (end 131.1275 80.645) (width 0.2) (layer "F.Cu") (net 1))
 (segment (start 131.1275 80.645) (end 131.1275 99.695) (width 0.2) (layer "B.Cu") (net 1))
 (segment (start 126.7855 44.5605) (end 136.02244 44.5605) (width 0.2) (layer "F.Cu") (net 3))
 (segment (start 122.70625 40.48125) (end 126.7855 44.5605) (width 0.2) (layer "F.Cu") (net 3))
 (segment (start 148.299376 34.8145) (end 152.4 38.915124) (width 0.2) (layer "F.Cu") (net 3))
 (segment (start 152.4 39.85) (end 154.78125 42.23125) (width 0.2) (layer "F.Cu") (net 3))
 (segment (start 136.02244 44.5605) (end 145.76844 34.8145) (width 0.2) (layer "F.Cu") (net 3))
 (segment (start 145.76844 34.8145) (end 148.299376 34.8145) (width 0.2) (layer "F.Cu") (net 3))
 (segment (start 152.4 38.915124) (end 152.4 39.85) (width 0.2) (layer "F.Cu") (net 3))
 (segment (start 146.20875 61.75375) (end 146.20875 48.5775) (width 0.2) (layer "F.Cu") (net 15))
 (segment (start 143.8275 64.135) (end 146.20875 61.75375) (width 0.2) (layer "F.Cu") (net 15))
 (segment (start 135.73125 72.23125) (end 135.73125 56.515) (width 0.2) (layer "F.Cu") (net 6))
 (segment (start 124.7775 83.185) (end 135.73125 72.23125) (width 0.2) (layer "F.Cu") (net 6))
 (segment (start 135.73125 56.515) (end 146.20875 46.0375) (width 0.2) (layer "F.Cu") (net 6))
 (segment (start 148.56075 44.77187) (end 147.28638 43.4975) (width 0.2) (layer "F.Cu") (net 7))
 (segment (start 147.28638 43.4975) (end 146.20875 43.4975) (width 0.2) (layer "F.Cu") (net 7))
 (segment (start 129.7265 80.064686) (end 141.915186 67.876) (width 0.2) (layer "F.Cu") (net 7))
 (segment (start 141.915186 67.876) (end 143.111684 67.876) (width 0.2) (layer "F.Cu") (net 7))
 (segment (start 131.686186 83.185) (end 129.7265 81.225314) (width 0.2) (layer "F.Cu") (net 7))
 (segment (start 143.111684 67.876) (end 148.56075 62.426934) (width 0.2) (layer "F.Cu") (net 7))
 (segment (start 129.7265 81.225314) (end 129.7265 80.064686) (width 0.2) (layer "F.Cu") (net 7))
 (segment (start 143.8275 83.185) (end 131.686186 83.185) (width 0.2) (layer "F.Cu") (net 7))
 (segment (start 148.56075 62.426934) (end 148.56075 44.77187) (width 0.2) (layer "F.Cu") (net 7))
 (segment (start 123.3765 82.604686) (end 135.33025 70.650936) (width 0.2) (layer "F.Cu") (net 2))
 (segment (start 124.7775 102.235) (end 124.7775 85.166314) (width 0.2) (layer "F.Cu") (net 2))
 (segment (start 135.33025 51.836) (end 146.20875 40.9575) (width 0.2) (layer "F.Cu") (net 2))
 (segment (start 123.3765 83.765314) (end 123.3765 82.604686) (width 0.2) (layer "F.Cu") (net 2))
 (segment (start 135.33025 70.650936) (end 135.33025 51.836) (width 0.2) (layer "F.Cu") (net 2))
 (segment (start 124.7775 85.166314) (end 123.3765 83.765314) (width 0.2) (layer "F.Cu") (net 2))
 (segment (start 124.7775 54.76875) (end 130.96875 48.5775) (width 0.2) (layer "F.Cu") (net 9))
 (segment (start 124.7775 64.135) (end 124.7775 54.76875) (width 0.2) (layer "F.Cu") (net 9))
 (segment (start 121.9055 104.87147) (end 121.9055 54.02312) (width 0.2) (layer "F.Cu") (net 10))
 (segment (start 129.89112 46.0375) (end 130.96875 46.0375) (width 0.2) (layer "F.Cu") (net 10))
 (segment (start 127.74597 102.235) (end 124.00497 105.976) (width 0.2) (layer "F.Cu") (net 10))
 (segment (start 124.00497 105.976) (end 123.01003 105.976) (width 0.2) (layer "F.Cu") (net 10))
 (segment (start 143.8275 102.235) (end 127.74597 102.235) (width 0.2) (layer "F.Cu") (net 10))
 (segment (start 123.01003 105.976) (end 121.9055 104.87147) (width 0.2) (layer "F.Cu") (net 10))
 (segment (start 121.9055 54.02312) (end 129.89112 46.0375) (width 0.2) (layer "F.Cu") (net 10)))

